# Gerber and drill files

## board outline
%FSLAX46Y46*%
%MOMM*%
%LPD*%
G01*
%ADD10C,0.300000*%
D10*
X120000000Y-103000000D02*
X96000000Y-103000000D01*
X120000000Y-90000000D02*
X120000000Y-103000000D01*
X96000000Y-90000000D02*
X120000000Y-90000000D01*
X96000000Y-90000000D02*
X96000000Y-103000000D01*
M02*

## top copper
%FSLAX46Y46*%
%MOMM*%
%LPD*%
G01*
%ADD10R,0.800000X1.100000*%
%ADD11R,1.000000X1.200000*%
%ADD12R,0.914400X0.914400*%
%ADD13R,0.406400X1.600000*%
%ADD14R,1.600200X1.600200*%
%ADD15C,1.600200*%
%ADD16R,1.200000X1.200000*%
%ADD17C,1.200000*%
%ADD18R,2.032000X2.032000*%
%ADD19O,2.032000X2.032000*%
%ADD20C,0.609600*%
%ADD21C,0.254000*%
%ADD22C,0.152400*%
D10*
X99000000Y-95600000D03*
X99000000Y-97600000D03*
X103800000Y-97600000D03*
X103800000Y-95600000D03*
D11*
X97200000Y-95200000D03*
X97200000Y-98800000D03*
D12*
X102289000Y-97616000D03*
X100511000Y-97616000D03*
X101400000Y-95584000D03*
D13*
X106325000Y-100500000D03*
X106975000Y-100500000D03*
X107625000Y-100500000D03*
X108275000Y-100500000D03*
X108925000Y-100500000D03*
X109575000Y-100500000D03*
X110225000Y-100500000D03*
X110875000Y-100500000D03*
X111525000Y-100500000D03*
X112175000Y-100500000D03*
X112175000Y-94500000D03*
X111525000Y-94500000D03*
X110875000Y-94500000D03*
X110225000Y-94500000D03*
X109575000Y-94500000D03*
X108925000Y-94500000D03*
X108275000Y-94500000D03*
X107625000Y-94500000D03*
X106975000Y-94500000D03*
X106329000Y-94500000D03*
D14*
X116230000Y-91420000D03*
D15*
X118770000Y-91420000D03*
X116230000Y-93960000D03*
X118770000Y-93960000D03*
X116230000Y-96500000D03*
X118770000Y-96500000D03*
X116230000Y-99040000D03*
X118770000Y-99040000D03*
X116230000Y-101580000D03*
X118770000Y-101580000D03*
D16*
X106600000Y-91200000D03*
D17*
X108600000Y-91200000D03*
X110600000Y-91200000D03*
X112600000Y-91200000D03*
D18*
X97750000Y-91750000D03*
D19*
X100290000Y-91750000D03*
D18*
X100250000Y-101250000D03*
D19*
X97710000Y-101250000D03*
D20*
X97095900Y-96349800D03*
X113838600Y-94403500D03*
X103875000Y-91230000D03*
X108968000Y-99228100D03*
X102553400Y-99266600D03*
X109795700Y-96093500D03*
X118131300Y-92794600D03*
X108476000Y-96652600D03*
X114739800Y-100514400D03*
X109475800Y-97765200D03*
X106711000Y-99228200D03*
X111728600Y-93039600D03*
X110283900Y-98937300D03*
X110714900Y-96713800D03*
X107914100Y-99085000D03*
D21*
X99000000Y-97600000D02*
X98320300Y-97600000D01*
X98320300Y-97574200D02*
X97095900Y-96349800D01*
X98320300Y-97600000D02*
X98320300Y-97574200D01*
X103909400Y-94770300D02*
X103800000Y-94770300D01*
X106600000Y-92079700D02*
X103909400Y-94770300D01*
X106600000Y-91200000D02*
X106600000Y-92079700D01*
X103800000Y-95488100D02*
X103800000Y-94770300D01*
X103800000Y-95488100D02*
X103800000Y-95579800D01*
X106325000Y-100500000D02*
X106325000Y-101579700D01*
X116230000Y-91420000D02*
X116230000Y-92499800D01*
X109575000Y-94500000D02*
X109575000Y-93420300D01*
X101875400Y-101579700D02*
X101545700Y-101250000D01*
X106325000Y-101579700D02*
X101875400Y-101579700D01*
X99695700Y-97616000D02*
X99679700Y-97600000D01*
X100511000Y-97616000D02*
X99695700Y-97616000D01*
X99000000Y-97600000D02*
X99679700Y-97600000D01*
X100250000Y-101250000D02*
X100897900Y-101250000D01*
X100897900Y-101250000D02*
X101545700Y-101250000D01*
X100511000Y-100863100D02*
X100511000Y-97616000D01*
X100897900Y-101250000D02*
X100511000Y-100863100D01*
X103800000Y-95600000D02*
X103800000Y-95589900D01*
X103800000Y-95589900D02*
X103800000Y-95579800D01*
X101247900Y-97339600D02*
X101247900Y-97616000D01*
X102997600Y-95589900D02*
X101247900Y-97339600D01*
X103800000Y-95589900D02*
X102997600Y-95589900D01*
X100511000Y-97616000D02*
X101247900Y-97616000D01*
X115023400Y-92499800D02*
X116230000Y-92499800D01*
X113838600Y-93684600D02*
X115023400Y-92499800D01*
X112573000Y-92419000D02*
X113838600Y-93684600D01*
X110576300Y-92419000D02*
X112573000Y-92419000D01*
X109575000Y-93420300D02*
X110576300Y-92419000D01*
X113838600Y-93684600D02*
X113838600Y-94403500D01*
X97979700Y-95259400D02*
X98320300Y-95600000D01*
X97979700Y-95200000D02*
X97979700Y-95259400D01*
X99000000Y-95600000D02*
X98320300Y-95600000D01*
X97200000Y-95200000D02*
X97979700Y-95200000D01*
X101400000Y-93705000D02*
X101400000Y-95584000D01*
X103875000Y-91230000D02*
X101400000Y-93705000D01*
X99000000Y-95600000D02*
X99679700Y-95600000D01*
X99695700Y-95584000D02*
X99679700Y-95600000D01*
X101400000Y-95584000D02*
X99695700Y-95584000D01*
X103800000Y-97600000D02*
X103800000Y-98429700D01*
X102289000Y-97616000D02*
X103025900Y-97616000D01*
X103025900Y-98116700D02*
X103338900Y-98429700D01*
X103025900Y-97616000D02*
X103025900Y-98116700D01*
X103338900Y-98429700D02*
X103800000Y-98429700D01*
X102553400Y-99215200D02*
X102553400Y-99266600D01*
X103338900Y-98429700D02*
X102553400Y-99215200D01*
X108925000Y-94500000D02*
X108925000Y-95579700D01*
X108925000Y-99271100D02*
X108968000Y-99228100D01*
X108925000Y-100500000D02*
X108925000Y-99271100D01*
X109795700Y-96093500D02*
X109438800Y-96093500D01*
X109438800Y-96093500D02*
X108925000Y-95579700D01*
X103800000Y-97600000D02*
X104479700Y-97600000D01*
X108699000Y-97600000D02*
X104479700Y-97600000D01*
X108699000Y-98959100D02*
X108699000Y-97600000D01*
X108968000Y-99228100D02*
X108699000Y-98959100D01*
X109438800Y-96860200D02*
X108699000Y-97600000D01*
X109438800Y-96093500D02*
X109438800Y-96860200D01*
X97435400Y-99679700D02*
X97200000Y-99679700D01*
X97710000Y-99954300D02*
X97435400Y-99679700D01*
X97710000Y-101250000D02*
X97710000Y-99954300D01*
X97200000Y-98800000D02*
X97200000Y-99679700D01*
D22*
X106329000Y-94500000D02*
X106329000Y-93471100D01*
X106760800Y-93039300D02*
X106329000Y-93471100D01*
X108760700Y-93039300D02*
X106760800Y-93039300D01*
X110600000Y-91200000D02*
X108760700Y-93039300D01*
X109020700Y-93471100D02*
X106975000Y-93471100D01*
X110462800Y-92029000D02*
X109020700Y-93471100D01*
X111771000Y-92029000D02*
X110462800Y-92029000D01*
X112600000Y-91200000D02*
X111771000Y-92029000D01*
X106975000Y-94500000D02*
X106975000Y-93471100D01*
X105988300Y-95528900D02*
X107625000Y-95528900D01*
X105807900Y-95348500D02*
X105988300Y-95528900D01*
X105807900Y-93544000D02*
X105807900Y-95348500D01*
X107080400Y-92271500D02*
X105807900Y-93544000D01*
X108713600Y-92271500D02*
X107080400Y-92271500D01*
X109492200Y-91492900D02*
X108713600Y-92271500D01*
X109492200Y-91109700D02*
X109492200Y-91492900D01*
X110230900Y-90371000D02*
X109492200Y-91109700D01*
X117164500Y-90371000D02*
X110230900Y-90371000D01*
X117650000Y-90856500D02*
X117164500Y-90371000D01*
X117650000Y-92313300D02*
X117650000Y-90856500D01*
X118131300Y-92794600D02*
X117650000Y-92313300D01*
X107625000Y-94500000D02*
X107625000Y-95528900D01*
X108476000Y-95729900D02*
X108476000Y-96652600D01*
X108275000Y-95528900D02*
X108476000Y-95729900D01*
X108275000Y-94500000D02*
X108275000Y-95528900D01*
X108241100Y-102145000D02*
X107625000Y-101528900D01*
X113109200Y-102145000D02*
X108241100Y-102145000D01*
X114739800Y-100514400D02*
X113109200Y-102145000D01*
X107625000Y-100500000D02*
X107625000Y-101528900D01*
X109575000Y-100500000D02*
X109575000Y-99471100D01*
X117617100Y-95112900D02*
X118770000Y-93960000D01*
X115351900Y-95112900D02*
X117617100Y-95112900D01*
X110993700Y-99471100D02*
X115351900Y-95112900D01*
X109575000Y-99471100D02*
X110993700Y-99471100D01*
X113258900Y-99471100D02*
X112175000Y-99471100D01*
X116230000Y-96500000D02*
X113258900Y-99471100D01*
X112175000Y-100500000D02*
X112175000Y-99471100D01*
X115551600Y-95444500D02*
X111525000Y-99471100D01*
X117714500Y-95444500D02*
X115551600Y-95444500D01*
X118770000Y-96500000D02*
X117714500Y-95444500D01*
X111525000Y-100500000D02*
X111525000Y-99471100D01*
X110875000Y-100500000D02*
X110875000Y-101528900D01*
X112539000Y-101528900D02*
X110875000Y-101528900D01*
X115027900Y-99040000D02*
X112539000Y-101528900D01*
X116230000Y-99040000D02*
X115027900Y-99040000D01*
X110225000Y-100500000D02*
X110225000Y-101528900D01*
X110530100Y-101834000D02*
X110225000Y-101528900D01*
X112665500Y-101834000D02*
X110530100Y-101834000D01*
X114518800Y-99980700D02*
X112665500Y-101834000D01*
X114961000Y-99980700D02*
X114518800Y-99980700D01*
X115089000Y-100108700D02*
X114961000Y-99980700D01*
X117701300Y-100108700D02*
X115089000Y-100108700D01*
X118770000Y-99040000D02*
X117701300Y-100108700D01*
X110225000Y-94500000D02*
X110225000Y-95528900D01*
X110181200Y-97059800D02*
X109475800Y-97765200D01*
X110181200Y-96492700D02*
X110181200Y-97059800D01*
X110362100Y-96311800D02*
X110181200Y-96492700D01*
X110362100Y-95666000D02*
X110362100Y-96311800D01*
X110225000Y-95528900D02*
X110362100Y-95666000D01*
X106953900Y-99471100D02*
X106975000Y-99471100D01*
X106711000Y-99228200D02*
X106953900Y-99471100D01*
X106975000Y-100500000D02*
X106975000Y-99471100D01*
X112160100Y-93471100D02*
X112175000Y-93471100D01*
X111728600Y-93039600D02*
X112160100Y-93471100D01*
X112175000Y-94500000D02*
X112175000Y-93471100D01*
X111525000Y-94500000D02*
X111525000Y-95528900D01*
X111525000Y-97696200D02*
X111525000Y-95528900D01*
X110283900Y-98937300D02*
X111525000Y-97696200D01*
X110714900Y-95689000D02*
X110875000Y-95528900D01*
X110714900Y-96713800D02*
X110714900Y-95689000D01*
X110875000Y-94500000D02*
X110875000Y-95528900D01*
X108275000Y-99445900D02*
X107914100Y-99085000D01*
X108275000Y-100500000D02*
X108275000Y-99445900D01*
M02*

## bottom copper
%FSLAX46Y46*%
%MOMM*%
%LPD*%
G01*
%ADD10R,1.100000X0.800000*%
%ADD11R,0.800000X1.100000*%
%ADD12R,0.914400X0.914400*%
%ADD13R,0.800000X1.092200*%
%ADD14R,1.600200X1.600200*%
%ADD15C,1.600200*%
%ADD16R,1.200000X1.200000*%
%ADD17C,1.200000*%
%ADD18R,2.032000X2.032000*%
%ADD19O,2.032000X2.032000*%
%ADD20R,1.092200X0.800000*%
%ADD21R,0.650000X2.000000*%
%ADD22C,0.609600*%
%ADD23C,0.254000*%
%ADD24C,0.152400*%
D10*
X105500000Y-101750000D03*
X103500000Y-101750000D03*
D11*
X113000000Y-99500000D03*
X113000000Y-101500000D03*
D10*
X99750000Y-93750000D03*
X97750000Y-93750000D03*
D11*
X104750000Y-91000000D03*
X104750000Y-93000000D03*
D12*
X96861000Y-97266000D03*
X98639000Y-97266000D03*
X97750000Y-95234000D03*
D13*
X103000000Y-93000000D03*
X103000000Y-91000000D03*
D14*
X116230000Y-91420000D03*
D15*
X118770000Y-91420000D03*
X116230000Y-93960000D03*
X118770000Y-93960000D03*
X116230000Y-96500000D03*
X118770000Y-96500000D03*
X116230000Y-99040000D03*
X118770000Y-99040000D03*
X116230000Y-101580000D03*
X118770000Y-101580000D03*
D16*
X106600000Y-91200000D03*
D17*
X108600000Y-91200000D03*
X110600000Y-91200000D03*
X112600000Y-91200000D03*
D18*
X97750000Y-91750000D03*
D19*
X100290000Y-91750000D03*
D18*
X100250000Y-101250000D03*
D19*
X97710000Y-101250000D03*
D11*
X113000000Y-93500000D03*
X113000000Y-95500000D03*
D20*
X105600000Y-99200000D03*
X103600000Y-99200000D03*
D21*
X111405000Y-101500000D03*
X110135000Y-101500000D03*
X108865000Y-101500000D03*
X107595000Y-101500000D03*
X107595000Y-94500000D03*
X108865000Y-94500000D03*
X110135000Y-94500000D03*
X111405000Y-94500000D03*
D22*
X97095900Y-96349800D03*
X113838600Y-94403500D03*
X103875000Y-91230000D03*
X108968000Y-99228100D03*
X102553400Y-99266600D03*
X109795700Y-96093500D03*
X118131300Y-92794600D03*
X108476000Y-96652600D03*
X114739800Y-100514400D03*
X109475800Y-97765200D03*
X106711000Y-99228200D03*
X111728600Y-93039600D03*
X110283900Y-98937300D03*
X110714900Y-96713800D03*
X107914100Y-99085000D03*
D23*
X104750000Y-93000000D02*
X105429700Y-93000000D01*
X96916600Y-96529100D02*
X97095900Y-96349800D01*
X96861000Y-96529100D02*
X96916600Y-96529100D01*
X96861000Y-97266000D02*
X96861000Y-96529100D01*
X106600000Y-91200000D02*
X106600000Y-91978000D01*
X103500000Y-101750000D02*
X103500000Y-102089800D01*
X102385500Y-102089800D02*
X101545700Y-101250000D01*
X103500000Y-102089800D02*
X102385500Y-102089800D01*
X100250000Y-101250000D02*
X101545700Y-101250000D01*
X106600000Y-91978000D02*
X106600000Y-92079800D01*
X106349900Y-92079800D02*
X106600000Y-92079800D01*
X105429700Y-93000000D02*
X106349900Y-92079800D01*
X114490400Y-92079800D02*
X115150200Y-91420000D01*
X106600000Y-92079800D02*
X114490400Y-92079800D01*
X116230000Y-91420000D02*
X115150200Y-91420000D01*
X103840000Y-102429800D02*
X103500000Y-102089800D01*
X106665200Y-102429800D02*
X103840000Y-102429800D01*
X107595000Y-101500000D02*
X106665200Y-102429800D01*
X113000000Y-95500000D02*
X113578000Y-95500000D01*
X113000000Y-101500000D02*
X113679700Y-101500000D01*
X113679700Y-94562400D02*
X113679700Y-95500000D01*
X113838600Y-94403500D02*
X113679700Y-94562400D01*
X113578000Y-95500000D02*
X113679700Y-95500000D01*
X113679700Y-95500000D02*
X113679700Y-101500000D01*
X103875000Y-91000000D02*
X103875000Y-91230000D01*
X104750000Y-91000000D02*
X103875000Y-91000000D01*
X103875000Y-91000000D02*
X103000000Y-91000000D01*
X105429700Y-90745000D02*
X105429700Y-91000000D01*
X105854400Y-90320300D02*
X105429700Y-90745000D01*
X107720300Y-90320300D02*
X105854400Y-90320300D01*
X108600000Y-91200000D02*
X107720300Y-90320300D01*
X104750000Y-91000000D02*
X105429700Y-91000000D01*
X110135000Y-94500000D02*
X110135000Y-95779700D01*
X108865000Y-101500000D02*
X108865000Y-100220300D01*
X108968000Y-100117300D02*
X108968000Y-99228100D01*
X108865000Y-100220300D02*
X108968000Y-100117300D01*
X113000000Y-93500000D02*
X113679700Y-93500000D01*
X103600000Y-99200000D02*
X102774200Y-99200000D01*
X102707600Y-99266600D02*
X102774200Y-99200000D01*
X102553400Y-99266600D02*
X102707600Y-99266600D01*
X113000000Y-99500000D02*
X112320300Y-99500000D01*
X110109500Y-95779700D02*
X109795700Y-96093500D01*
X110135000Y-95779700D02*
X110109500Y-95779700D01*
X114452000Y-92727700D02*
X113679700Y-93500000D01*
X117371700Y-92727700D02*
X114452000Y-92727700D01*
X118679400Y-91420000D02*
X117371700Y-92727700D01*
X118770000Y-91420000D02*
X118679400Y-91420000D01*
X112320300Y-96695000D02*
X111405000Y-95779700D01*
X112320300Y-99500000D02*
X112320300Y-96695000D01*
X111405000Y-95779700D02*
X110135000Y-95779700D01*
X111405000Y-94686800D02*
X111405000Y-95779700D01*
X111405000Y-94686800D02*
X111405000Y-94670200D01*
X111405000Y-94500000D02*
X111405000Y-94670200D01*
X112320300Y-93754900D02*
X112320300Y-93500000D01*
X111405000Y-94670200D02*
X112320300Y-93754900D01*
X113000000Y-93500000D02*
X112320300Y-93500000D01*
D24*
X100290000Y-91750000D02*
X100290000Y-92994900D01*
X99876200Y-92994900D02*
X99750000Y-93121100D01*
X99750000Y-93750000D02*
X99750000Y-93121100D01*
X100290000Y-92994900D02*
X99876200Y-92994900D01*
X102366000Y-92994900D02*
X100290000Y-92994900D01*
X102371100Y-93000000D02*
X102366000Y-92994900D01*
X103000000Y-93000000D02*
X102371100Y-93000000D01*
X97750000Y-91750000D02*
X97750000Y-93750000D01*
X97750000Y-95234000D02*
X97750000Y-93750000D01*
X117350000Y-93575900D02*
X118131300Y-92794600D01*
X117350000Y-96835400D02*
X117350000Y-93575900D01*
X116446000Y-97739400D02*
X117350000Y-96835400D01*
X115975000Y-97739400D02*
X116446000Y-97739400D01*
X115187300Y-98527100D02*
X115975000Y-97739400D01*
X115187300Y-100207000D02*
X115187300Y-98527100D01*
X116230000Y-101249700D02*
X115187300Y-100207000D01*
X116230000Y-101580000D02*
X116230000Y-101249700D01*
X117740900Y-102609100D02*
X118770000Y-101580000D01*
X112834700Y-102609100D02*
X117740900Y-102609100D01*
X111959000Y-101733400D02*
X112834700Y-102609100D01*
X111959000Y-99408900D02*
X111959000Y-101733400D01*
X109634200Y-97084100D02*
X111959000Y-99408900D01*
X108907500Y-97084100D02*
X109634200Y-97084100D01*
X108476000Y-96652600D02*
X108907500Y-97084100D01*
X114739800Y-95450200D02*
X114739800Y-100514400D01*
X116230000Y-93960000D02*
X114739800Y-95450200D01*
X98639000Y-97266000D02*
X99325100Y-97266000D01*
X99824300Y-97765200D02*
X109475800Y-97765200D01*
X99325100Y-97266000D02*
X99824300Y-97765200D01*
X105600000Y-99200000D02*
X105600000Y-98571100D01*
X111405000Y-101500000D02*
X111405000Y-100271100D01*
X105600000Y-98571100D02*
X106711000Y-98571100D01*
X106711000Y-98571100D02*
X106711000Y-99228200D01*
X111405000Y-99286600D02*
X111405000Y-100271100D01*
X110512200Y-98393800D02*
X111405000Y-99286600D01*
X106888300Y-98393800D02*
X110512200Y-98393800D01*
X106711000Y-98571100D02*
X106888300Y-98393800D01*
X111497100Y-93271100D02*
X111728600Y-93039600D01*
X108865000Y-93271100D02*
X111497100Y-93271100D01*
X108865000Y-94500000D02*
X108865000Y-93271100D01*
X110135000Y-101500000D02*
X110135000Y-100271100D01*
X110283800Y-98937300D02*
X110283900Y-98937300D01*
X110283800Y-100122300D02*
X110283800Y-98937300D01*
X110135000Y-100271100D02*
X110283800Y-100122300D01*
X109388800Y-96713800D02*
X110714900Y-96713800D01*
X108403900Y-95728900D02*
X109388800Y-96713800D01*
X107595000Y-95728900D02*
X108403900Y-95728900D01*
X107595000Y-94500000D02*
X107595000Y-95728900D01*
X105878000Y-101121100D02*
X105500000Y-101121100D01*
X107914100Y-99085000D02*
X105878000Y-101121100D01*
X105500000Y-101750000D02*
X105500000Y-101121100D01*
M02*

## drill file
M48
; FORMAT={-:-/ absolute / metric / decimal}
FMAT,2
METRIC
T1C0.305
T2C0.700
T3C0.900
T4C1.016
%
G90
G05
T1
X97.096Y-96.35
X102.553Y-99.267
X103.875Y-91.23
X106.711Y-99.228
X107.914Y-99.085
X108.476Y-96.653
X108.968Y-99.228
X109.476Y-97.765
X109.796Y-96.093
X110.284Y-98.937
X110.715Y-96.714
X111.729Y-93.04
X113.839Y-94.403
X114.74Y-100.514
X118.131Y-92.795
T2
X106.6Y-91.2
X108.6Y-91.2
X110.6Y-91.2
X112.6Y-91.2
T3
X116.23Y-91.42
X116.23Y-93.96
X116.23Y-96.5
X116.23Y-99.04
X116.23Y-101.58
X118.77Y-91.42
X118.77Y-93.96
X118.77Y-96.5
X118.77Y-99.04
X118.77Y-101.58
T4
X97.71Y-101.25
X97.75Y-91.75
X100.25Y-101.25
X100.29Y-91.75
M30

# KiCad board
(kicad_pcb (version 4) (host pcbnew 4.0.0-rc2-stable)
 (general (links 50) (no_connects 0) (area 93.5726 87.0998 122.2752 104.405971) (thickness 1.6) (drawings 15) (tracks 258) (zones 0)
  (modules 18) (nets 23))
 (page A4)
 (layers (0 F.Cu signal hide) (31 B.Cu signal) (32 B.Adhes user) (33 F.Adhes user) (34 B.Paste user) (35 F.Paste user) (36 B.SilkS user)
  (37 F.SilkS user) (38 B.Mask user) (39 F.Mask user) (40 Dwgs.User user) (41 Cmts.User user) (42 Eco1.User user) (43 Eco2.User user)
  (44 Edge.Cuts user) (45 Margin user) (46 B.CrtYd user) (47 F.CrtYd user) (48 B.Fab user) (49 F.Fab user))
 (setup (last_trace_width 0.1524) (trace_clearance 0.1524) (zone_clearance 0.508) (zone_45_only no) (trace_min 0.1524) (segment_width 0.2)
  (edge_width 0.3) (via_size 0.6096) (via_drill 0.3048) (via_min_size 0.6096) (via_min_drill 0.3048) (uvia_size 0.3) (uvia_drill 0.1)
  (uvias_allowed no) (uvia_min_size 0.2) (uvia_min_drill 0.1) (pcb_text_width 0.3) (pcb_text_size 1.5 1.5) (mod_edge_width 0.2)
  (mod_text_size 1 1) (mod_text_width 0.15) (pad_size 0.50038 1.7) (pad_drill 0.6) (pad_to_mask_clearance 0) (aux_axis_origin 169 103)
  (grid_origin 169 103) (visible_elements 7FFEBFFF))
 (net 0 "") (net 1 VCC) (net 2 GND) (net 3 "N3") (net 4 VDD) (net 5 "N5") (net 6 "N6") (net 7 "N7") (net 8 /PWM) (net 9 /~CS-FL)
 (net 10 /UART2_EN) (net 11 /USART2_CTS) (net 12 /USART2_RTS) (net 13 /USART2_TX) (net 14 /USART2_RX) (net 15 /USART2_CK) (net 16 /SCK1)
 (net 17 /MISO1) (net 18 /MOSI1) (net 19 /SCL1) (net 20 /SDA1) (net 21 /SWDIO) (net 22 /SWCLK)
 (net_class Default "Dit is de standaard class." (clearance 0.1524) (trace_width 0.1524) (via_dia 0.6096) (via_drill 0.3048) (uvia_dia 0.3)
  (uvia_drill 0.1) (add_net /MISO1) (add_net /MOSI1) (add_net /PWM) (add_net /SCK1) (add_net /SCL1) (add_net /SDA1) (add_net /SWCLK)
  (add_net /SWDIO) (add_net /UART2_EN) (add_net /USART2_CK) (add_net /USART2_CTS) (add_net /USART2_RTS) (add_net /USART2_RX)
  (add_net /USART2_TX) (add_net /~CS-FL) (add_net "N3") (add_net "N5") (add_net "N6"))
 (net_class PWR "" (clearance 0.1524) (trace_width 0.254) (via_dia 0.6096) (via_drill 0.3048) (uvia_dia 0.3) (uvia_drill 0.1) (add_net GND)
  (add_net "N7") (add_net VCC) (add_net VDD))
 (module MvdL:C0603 (layer F.Cu) (at 99 96.6 270)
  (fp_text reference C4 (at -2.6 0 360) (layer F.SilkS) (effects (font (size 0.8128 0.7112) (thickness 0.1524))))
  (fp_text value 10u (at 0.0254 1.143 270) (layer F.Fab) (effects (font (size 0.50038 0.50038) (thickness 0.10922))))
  (pad 1 smd rect (at -1 0 270) (size 1.1 0.8) (layers F.Cu F.Paste F.Mask) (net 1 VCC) (clearance 0.1524))
  (pad 2 smd rect (at 1 0 270) (size 1.1 0.8) (layers F.Cu F.Paste F.Mask) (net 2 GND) (clearance 0.1524)))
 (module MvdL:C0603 (layer B.Cu) (at 104.5 101.75 180)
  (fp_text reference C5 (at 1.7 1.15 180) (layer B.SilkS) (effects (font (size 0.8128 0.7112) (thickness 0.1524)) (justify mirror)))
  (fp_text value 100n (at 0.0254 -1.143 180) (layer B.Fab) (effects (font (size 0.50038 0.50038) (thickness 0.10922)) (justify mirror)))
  (pad 1 smd rect (at -1 0 180) (size 1.1 0.8) (layers B.Cu B.Paste B.Mask) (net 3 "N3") (clearance 0.1524))
  (pad 2 smd rect (at 1 0 180) (size 1.1 0.8) (layers B.Cu B.Paste B.Mask) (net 2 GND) (clearance 0.1524)))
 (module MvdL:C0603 (layer F.Cu) (at 103.8 96.6 90)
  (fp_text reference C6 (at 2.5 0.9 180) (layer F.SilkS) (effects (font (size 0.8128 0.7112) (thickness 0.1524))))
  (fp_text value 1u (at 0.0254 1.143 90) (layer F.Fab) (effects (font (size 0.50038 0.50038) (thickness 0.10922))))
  (pad 1 smd rect (at -1 0 90) (size 1.1 0.8) (layers F.Cu F.Paste F.Mask) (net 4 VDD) (clearance 0.1524))
  (pad 2 smd rect (at 1 0 90) (size 1.1 0.8) (layers F.Cu F.Paste F.Mask) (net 2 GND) (clearance 0.1524)))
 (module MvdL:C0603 (layer B.Cu) (at 113 100.5 270)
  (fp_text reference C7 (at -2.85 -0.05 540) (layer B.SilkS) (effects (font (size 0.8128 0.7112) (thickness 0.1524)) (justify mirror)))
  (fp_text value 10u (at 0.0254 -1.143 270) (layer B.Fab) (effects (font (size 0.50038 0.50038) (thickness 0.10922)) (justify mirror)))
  (pad 1 smd rect (at -1 0 270) (size 1.1 0.8) (layers B.Cu B.Paste B.Mask) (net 4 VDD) (clearance 0.1524))
  (pad 2 smd rect (at 1 0 270) (size 1.1 0.8) (layers B.Cu B.Paste B.Mask) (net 2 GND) (clearance 0.1524)))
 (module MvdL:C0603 (layer B.Cu) (at 98.75 93.75 180)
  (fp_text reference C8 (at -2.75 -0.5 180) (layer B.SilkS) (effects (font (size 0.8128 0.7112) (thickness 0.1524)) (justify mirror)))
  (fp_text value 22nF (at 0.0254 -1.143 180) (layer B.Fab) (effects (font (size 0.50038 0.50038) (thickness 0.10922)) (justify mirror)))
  (pad 1 smd rect (at -1 0 180) (size 1.1 0.8) (layers B.Cu B.Paste B.Mask) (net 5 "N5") (clearance 0.1524))
  (pad 2 smd rect (at 1 0 180) (size 1.1 0.8) (layers B.Cu B.Paste B.Mask) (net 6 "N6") (clearance 0.1524)))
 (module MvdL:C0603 (layer B.Cu) (at 104.75 92 270)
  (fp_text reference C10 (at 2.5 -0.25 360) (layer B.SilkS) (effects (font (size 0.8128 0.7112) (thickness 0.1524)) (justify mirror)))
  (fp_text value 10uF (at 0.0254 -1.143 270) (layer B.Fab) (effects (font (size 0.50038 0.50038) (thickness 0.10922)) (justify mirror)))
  (pad 1 smd rect (at -1 0 270) (size 1.1 0.8) (layers B.Cu B.Paste B.Mask) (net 1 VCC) (clearance 0.1524))
  (pad 2 smd rect (at 1 0 270) (size 1.1 0.8) (layers B.Cu B.Paste B.Mask) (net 2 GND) (clearance 0.1524)))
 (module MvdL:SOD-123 (layer F.Cu) (at 97.2 97 270)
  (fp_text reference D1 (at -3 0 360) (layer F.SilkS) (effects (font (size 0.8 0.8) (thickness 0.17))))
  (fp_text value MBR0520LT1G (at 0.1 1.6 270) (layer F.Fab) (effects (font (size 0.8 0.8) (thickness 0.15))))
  (pad C smd rect (at -1.8 0 270) (size 1.2 1) (layers F.Cu F.Paste F.Mask) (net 1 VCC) (clearance 0.1524))
  (pad A smd rect (at 1.8 0 270) (size 1.2 1) (layers F.Cu F.Paste F.Mask) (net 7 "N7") (clearance 0.1524)))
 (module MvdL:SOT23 (layer B.Cu) (at 97.75 96.25)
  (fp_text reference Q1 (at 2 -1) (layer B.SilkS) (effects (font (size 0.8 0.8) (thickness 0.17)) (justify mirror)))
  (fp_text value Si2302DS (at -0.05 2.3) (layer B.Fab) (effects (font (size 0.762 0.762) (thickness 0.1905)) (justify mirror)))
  (pad 2 smd rect (at -0.889 1.016) (size 0.9144 0.9144) (layers B.Cu B.Paste B.Mask) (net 2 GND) (die_length -2147.483648)
   (clearance 0.1524))
  (pad 1 smd rect (at 0.889 1.016) (size 0.9144 0.9144) (layers B.Cu B.Paste B.Mask) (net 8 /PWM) (clearance 0.1524))
  (pad 3 smd rect (at 0 -1.016) (size 0.9144 0.9144) (layers B.Cu B.Paste B.Mask) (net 6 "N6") (clearance 0.1524)))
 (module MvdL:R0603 (layer B.Cu) (at 103 92 90)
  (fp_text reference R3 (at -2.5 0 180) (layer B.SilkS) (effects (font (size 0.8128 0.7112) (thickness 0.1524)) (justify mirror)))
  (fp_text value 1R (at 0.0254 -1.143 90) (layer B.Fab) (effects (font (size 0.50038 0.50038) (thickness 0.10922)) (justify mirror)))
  (pad 1 smd rect (at -1 0 90) (size 1.0922 0.8) (layers B.Cu B.Paste B.Mask) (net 5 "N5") (clearance 0.1524))
  (pad 2 smd rect (at 1 0 90) (size 1.0922 0.8) (layers B.Cu B.Paste B.Mask) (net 1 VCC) (clearance 0.1524)))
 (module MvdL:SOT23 (layer F.Cu) (at 101.4 96.6 180)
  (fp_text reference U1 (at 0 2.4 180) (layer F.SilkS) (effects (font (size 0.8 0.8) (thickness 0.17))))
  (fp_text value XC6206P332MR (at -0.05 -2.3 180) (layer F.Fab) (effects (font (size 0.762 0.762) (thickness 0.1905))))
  (pad 2 smd rect (at -0.889 -1.016 180) (size 0.9144 0.9144) (layers F.Cu F.Paste F.Mask) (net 4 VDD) (die_length -2147.483648)
   (clearance 0.1524))
  (pad 1 smd rect (at 0.889 -1.016 180) (size 0.9144 0.9144) (layers F.Cu F.Paste F.Mask) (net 2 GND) (clearance 0.1524))
  (pad 3 smd rect (at 0 1.016 180) (size 0.9144 0.9144) (layers F.Cu F.Paste F.Mask) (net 1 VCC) (clearance 0.1524)))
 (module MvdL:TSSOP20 (layer F.Cu) (at 109.25 97.5)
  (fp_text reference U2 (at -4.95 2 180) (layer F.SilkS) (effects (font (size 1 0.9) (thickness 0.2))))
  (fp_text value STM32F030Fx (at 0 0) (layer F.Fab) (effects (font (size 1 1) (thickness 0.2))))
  (pad 1 smd rect (at -2.925 3) (size 0.4064 1.6) (layers F.Cu F.Paste F.Mask) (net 2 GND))
  (pad 2 smd rect (at -2.275 3) (size 0.4064 1.6) (layers F.Cu F.Paste F.Mask) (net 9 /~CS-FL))
  (pad 3 smd rect (at -1.625 3) (size 0.4064 1.6) (layers F.Cu F.Paste F.Mask) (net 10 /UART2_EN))
  (pad 4 smd rect (at -0.975 3) (size 0.4064 1.6) (layers F.Cu F.Paste F.Mask) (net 3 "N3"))
  (pad 5 smd rect (at -0.325 3) (size 0.4064 1.6) (layers F.Cu F.Paste F.Mask) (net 4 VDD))
  (pad 6 smd rect (at 0.325 3) (size 0.4064 1.6) (layers F.Cu F.Paste F.Mask) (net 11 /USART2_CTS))
  (pad 7 smd rect (at 0.975 3) (size 0.4064 1.6) (layers F.Cu F.Paste F.Mask) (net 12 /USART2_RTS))
  (pad 8 smd rect (at 1.625 3) (size 0.4064 1.6) (layers F.Cu F.Paste F.Mask) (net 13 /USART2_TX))
  (pad 9 smd rect (at 2.275 3) (size 0.4064 1.6) (layers F.Cu F.Paste F.Mask) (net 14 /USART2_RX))
  (pad 10 smd rect (at 2.925 3) (size 0.4064 1.6) (layers F.Cu F.Paste F.Mask) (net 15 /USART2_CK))
  (pad 11 smd rect (at 2.925 -3) (size 0.4064 1.6) (layers F.Cu F.Paste F.Mask) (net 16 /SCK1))
  (pad 12 smd rect (at 2.275 -3) (size 0.4064 1.6) (layers F.Cu F.Paste F.Mask) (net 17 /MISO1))
  (pad 13 smd rect (at 1.625 -3) (size 0.4064 1.6) (layers F.Cu F.Paste F.Mask) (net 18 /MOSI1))
  (pad 14 smd rect (at 0.975 -3) (size 0.4064 1.6) (layers F.Cu F.Paste F.Mask) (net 8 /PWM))
  (pad 15 smd rect (at 0.325 -3) (size 0.4064 1.6) (layers F.Cu F.Paste F.Mask) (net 2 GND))
  (pad 16 smd rect (at -0.325 -3) (size 0.4064 1.6) (layers F.Cu F.Paste F.Mask) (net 4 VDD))
  (pad 17 smd rect (at -0.975 -3) (size 0.4064 1.6) (layers F.Cu F.Paste F.Mask) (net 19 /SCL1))
  (pad 18 smd rect (at -1.625 -3) (size 0.4064 1.6) (layers F.Cu F.Paste F.Mask) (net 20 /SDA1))
  (pad 19 smd rect (at -2.275 -3) (size 0.4064 1.6) (layers F.Cu F.Paste F.Mask) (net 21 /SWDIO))
  (pad 20 smd rect (at -2.921 -3) (size 0.4064 1.6) (layers F.Cu F.Paste F.Mask) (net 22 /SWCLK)))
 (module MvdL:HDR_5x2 (layer F.Cu) (at 117.5 96.5 270)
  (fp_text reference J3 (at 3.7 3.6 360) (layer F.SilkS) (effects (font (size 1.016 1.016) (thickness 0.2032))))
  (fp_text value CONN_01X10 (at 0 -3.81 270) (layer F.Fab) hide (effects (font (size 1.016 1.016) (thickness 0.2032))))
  (pad 1 thru_hole rect (at -5.08 1.27 270) (size 1.6002 1.6002) (drill 0.9) (layers *.Cu *.Mask F.SilkS) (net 2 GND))
  (pad 2 thru_hole circle (at -5.08 -1.27 270) (size 1.6002 1.6002) (drill 0.9) (layers *.Cu *.Mask F.SilkS) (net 4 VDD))
  (pad 3 thru_hole circle (at -2.54 1.27 270) (size 1.6002 1.6002) (drill 0.9) (layers *.Cu *.Mask F.SilkS) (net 10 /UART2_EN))
  (pad 4 thru_hole circle (at -2.54 -1.27 270) (size 1.6002 1.6002) (drill 0.9) (layers *.Cu *.Mask F.SilkS) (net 11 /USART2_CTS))
  (pad 5 thru_hole circle (at 0 1.27 270) (size 1.6002 1.6002) (drill 0.9) (layers *.Cu *.Mask F.SilkS) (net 15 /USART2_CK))
  (pad 6 thru_hole circle (at 0 -1.27 270) (size 1.6002 1.6002) (drill 0.9) (layers *.Cu *.Mask F.SilkS) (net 14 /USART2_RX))
  (pad 7 thru_hole circle (at 2.54 1.27 270) (size 1.6002 1.6002) (drill 0.9) (layers *.Cu *.Mask F.SilkS) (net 13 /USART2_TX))
  (pad 8 thru_hole circle (at 2.54 -1.27 270) (size 1.6002 1.6002) (drill 0.9) (layers *.Cu *.Mask F.SilkS) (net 12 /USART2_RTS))
  (pad 9 thru_hole circle (at 5.08 1.27 270) (size 1.6002 1.6002) (drill 0.9) (layers *.Cu *.Mask F.SilkS) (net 20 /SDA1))
  (pad 10 thru_hole circle (at 5.08 -1.27 270) (size 1.6002 1.6002) (drill 0.9) (layers *.Cu *.Mask F.SilkS) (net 19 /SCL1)))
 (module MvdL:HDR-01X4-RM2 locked (layer F.Cu) (at 106.6 91.2)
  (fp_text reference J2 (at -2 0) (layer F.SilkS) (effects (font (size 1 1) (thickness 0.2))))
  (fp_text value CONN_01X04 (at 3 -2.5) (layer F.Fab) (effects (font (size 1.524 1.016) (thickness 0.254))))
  (pad 1 thru_hole rect (at 0 0) (size 1.2 1.2) (drill 0.7) (layers *.Cu *.Mask F.SilkS) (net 2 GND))
  (pad 2 thru_hole circle (at 2 0) (size 1.2 1.2) (drill 0.7) (layers *.Cu *.Mask F.SilkS) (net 1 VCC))
  (pad 3 thru_hole circle (at 4 0) (size 1.2 1.2) (drill 0.7) (layers *.Cu *.Mask F.SilkS) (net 22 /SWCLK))
  (pad 4 thru_hole circle (at 6 0) (size 1.2 1.2) (drill 0.7) (layers *.Cu *.Mask F.SilkS) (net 21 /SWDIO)))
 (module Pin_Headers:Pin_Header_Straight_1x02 (layer F.Cu) (at 97.75 91.75 90)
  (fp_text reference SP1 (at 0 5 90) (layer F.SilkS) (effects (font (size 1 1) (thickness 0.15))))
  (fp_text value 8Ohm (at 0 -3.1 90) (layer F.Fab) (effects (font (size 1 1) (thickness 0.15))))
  (pad 1 thru_hole rect (at 0 0 90) (size 2.032 2.032) (drill 1.016) (layers *.Cu *.Mask F.SilkS) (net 6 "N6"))
  (pad 2 thru_hole oval (at 0 2.54 90) (size 2.032 2.032) (drill 1.016) (layers *.Cu *.Mask F.SilkS) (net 5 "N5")))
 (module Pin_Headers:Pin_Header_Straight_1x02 (layer F.Cu) (at 100.25 101.25 270)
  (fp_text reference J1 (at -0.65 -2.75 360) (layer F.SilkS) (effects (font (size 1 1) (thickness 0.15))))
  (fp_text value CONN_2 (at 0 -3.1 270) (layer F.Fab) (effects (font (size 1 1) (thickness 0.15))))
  (pad 1 thru_hole rect (at 0 0 270) (size 2.032 2.032) (drill 1.016) (layers *.Cu *.Mask F.SilkS) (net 2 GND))
  (pad 2 thru_hole oval (at 0 2.54 270) (size 2.032 2.032) (drill 1.016) (layers *.Cu *.Mask F.SilkS) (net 7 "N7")))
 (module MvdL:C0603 (layer B.Cu) (at 113 94.5 270)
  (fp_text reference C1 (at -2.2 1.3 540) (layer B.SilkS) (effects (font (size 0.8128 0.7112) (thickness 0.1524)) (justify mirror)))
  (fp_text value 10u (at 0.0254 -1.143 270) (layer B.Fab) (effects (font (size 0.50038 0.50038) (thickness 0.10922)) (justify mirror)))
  (pad 1 smd rect (at -1 0 270) (size 1.1 0.8) (layers B.Cu B.Paste B.Mask) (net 4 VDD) (clearance 0.1524))
  (pad 2 smd rect (at 1 0 270) (size 1.1 0.8) (layers B.Cu B.Paste B.Mask) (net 2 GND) (clearance 0.1524)))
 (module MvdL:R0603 (layer B.Cu) (at 104.6 99.2 180)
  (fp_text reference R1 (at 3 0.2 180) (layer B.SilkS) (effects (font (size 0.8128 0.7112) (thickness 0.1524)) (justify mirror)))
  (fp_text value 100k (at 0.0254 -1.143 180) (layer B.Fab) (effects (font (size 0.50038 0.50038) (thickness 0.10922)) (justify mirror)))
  (pad 1 smd rect (at -1 0 180) (size 1.0922 0.8) (layers B.Cu B.Paste B.Mask) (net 9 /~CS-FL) (clearance 0.1524))
  (pad 2 smd rect (at 1 0 180) (size 1.0922 0.8) (layers B.Cu B.Paste B.Mask) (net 4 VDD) (clearance 0.1524)))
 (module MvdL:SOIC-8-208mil (layer B.Cu) (at 109.5 98 90)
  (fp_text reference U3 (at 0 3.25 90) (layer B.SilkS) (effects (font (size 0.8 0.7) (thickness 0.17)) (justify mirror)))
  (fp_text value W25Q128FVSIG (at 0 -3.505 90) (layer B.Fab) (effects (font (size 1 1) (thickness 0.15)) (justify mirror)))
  (pad 1 smd rect (at -3.5 1.905 90) (size 2 0.65) (layers B.Cu B.Paste B.Mask) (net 9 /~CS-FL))
  (pad 2 smd rect (at -3.5 0.635 90) (size 2 0.65) (layers B.Cu B.Paste B.Mask) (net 17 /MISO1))
  (pad 3 smd rect (at -3.5 -0.635 90) (size 2 0.65) (layers B.Cu B.Paste B.Mask) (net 4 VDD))
  (pad 4 smd rect (at -3.5 -1.905 90) (size 2 0.65) (layers B.Cu B.Paste B.Mask) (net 2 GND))
  (pad 5 smd rect (at 3.5 -1.905 90) (size 2 0.65) (layers B.Cu B.Paste B.Mask) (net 18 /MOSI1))
  (pad 6 smd rect (at 3.5 -0.635 90) (size 2 0.65) (layers B.Cu B.Paste B.Mask) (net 16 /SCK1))
  (pad 7 smd rect (at 3.5 0.635 90) (size 2 0.65) (layers B.Cu B.Paste B.Mask) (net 4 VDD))
  (pad 8 smd rect (at 3.5 1.905 90) (size 2 0.65) (layers B.Cu B.Paste B.Mask) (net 4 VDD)))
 (gr_line (start 120 103) (end 96 103) (angle 90) (layer Edge.Cuts) (width 0.3))
 (gr_line (start 120 90) (end 120 103) (angle 90) (layer Edge.Cuts) (width 0.3))
 (gr_line (start 96 90) (end 120 90) (angle 90) (layer Edge.Cuts) (width 0.3))
 (gr_line (start 96 90) (end 96 103) (angle 90) (layer Edge.Cuts) (width 0.3))
 (via (at 97.0959 96.3498) (size 0.6096) (layers F.Cu B.Cu) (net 2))
 (via (at 113.8386 94.4035) (size 0.6096) (layers F.Cu B.Cu) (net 2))
 (segment (start 104.75 93) (end 105.4297 93) (width 0.254) (layer B.Cu) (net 2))
 (segment (start 99 97.6) (end 98.3203 97.6) (width 0.254) (layer F.Cu) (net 2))
 (segment (start 96.9166 96.5291) (end 97.0959 96.3498) (width 0.254) (layer B.Cu) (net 2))
 (segment (start 96.861 96.5291) (end 96.9166 96.5291) (width 0.254) (layer B.Cu) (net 2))
 (segment (start 98.3203 97.5742) (end 97.0959 96.3498) (width 0.254) (layer F.Cu) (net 2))
 (segment (start 98.3203 97.6) (end 98.3203 97.5742) (width 0.254) (layer F.Cu) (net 2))
 (segment (start 96.861 97.266) (end 96.861 96.5291) (width 0.254) (layer B.Cu) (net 2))
 (segment (start 103.9094 94.7703) (end 103.8 94.7703) (width 0.254) (layer F.Cu) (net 2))
 (segment (start 106.6 92.0797) (end 103.9094 94.7703) (width 0.254) (layer F.Cu) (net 2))
 (segment (start 106.6 91.2) (end 106.6 92.0797) (width 0.254) (layer F.Cu) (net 2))
 (segment (start 103.8 95.4881) (end 103.8 94.7703) (width 0.254) (layer F.Cu) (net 2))
 (segment (start 103.8 95.4881) (end 103.8 95.5798) (width 0.254) (layer F.Cu) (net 2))
 (segment (start 106.325 100.5) (end 106.325 101.5797) (width 0.254) (layer F.Cu) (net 2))
 (segment (start 106.6 91.2) (end 106.6 91.978) (width 0.254) (layer B.Cu) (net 2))
 (segment (start 116.23 91.42) (end 116.23 92.4998) (width 0.254) (layer F.Cu) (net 2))
 (segment (start 103.5 101.75) (end 103.5 102.0898) (width 0.254) (layer B.Cu) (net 2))
 (segment (start 102.3855 102.0898) (end 101.5457 101.25) (width 0.254) (layer B.Cu) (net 2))
 (segment (start 103.5 102.0898) (end 102.3855 102.0898) (width 0.254) (layer B.Cu) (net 2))
 (segment (start 100.25 101.25) (end 101.5457 101.25) (width 0.254) (layer B.Cu) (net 2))
 (segment (start 109.575 94.5) (end 109.575 93.4203) (width 0.254) (layer F.Cu) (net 2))
 (segment (start 106.6 91.978) (end 106.6 92.0798) (width 0.254) (layer B.Cu) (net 2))
 (segment (start 106.3499 92.0798) (end 106.6 92.0798) (width 0.254) (layer B.Cu) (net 2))
 (segment (start 105.4297 93) (end 106.3499 92.0798) (width 0.254) (layer B.Cu) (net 2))
 (segment (start 114.4904 92.0798) (end 115.1502 91.42) (width 0.254) (layer B.Cu) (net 2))
 (segment (start 106.6 92.0798) (end 114.4904 92.0798) (width 0.254) (layer B.Cu) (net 2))
 (segment (start 116.23 91.42) (end 115.1502 91.42) (width 0.254) (layer B.Cu) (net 2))
 (segment (start 103.84 102.4298) (end 103.5 102.0898) (width 0.254) (layer B.Cu) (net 2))
 (segment (start 106.6652 102.4298) (end 103.84 102.4298) (width 0.254) (layer B.Cu) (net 2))
 (segment (start 107.595 101.5) (end 106.6652 102.4298) (width 0.254) (layer B.Cu) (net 2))
 (segment (start 113 95.5) (end 113.578 95.5) (width 0.254) (layer B.Cu) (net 2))
 (segment (start 113 101.5) (end 113.6797 101.5) (width 0.254) (layer B.Cu) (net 2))
 (segment (start 101.8754 101.5797) (end 101.5457 101.25) (width 0.254) (layer F.Cu) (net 2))
 (segment (start 106.325 101.5797) (end 101.8754 101.5797) (width 0.254) (layer F.Cu) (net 2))
 (segment (start 99.6957 97.616) (end 99.6797 97.6) (width 0.254) (layer F.Cu) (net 2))
 (segment (start 100.511 97.616) (end 99.6957 97.616) (width 0.254) (layer F.Cu) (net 2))
 (segment (start 99 97.6) (end 99.6797 97.6) (width 0.254) (layer F.Cu) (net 2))
 (segment (start 100.25 101.25) (end 100.8979 101.25) (width 0.254) (layer F.Cu) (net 2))
 (segment (start 100.8979 101.25) (end 101.5457 101.25) (width 0.254) (layer F.Cu) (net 2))
 (segment (start 100.511 100.8631) (end 100.511 97.616) (width 0.254) (layer F.Cu) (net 2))
 (segment (start 100.8979 101.25) (end 100.511 100.8631) (width 0.254) (layer F.Cu) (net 2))
 (segment (start 103.8 95.6) (end 103.8 95.5899) (width 0.254) (layer F.Cu) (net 2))
 (segment (start 103.8 95.5899) (end 103.8 95.5798) (width 0.254) (layer F.Cu) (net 2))
 (segment (start 101.2479 97.3396) (end 101.2479 97.616) (width 0.254) (layer F.Cu) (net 2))
 (segment (start 102.9976 95.5899) (end 101.2479 97.3396) (width 0.254) (layer F.Cu) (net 2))
 (segment (start 103.8 95.5899) (end 102.9976 95.5899) (width 0.254) (layer F.Cu) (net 2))
 (segment (start 100.511 97.616) (end 101.2479 97.616) (width 0.254) (layer F.Cu) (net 2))
 (segment (start 113.6797 94.5624) (end 113.6797 95.5) (width 0.254) (layer B.Cu) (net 2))
 (segment (start 113.8386 94.4035) (end 113.6797 94.5624) (width 0.254) (layer B.Cu) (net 2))
 (segment (start 113.578 95.5) (end 113.6797 95.5) (width 0.254) (layer B.Cu) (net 2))
 (segment (start 113.6797 95.5) (end 113.6797 101.5) (width 0.254) (layer B.Cu) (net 2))
 (segment (start 115.0234 92.4998) (end 116.23 92.4998) (width 0.254) (layer F.Cu) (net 2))
 (segment (start 113.8386 93.6846) (end 115.0234 92.4998) (width 0.254) (layer F.Cu) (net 2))
 (segment (start 112.573 92.419) (end 113.8386 93.6846) (width 0.254) (layer F.Cu) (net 2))
 (segment (start 110.5763 92.419) (end 112.573 92.419) (width 0.254) (layer F.Cu) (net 2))
 (segment (start 109.575 93.4203) (end 110.5763 92.419) (width 0.254) (layer F.Cu) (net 2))
 (segment (start 113.8386 93.6846) (end 113.8386 94.4035) (width 0.254) (layer F.Cu) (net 2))
 (via (at 103.875 91.23) (size 0.6096) (layers F.Cu B.Cu) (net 1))
 (segment (start 97.9797 95.2594) (end 98.3203 95.6) (width 0.254) (layer F.Cu) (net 1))
 (segment (start 97.9797 95.2) (end 97.9797 95.2594) (width 0.254) (layer F.Cu) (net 1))
 (segment (start 99 95.6) (end 98.3203 95.6) (width 0.254) (layer F.Cu) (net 1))
 (segment (start 97.2 95.2) (end 97.9797 95.2) (width 0.254) (layer F.Cu) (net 1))
 (segment (start 103.875 91) (end 103.875 91.23) (width 0.254) (layer B.Cu) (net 1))
 (segment (start 104.75 91) (end 103.875 91) (width 0.254) (layer B.Cu) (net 1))
 (segment (start 103.875 91) (end 103 91) (width 0.254) (layer B.Cu) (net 1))
 (segment (start 101.4 93.705) (end 101.4 95.584) (width 0.254) (layer F.Cu) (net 1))
 (segment (start 103.875 91.23) (end 101.4 93.705) (width 0.254) (layer F.Cu) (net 1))
 (segment (start 99 95.6) (end 99.6797 95.6) (width 0.254) (layer F.Cu) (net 1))
 (segment (start 99.6957 95.584) (end 99.6797 95.6) (width 0.254) (layer F.Cu) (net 1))
 (segment (start 101.4 95.584) (end 99.6957 95.584) (width 0.254) (layer F.Cu) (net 1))
 (segment (start 105.4297 90.745) (end 105.4297 91) (width 0.254) (layer B.Cu) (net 1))
 (segment (start 105.8544 90.3203) (end 105.4297 90.745) (width 0.254) (layer B.Cu) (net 1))
 (segment (start 107.7203 90.3203) (end 105.8544 90.3203) (width 0.254) (layer B.Cu) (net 1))
 (segment (start 108.6 91.2) (end 107.7203 90.3203) (width 0.254) (layer B.Cu) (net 1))
 (segment (start 104.75 91) (end 105.4297 91) (width 0.254) (layer B.Cu) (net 1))
 (via (at 108.968 99.2281) (size 0.6096) (layers F.Cu B.Cu) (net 4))
 (via (at 102.5534 99.2666) (size 0.6096) (layers F.Cu B.Cu) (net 4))
 (via (at 109.7957 96.0935) (size 0.6096) (layers F.Cu B.Cu) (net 4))
 (segment (start 110.135 94.5) (end 110.135 95.7797) (width 0.254) (layer B.Cu) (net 4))
 (segment (start 108.865 101.5) (end 108.865 100.2203) (width 0.254) (layer B.Cu) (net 4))
 (segment (start 108.968 100.1173) (end 108.968 99.2281) (width 0.254) (layer B.Cu) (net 4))
 (segment (start 108.865 100.2203) (end 108.968 100.1173) (width 0.254) (layer B.Cu) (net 4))
 (segment (start 113 93.5) (end 113.6797 93.5) (width 0.254) (layer B.Cu) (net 4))
 (segment (start 103.8 97.6) (end 103.8 98.4297) (width 0.254) (layer F.Cu) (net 4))
 (segment (start 102.289 97.616) (end 103.0259 97.616) (width 0.254) (layer F.Cu) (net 4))
 (segment (start 103.0259 98.1167) (end 103.3389 98.4297) (width 0.254) (layer F.Cu) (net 4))
 (segment (start 103.0259 97.616) (end 103.0259 98.1167) (width 0.254) (layer F.Cu) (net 4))
 (segment (start 103.3389 98.4297) (end 103.8 98.4297) (width 0.254) (layer F.Cu) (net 4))
 (segment (start 103.6 99.2) (end 102.7742 99.2) (width 0.254) (layer B.Cu) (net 4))
 (segment (start 102.7076 99.2666) (end 102.7742 99.2) (width 0.254) (layer B.Cu) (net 4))
 (segment (start 102.5534 99.2666) (end 102.7076 99.2666) (width 0.254) (layer B.Cu) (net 4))
 (segment (start 102.5534 99.2152) (end 102.5534 99.2666) (width 0.254) (layer F.Cu) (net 4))
 (segment (start 103.3389 98.4297) (end 102.5534 99.2152) (width 0.254) (layer F.Cu) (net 4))
 (segment (start 113 99.5) (end 112.3203 99.5) (width 0.254) (layer B.Cu) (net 4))
 (segment (start 110.1095 95.7797) (end 109.7957 96.0935) (width 0.254) (layer B.Cu) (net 4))
 (segment (start 110.135 95.7797) (end 110.1095 95.7797) (width 0.254) (layer B.Cu) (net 4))
 (segment (start 108.925 94.5) (end 108.925 95.5797) (width 0.254) (layer F.Cu) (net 4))
 (segment (start 108.925 99.2711) (end 108.968 99.2281) (width 0.254) (layer F.Cu) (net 4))
 (segment (start 108.925 100.5) (end 108.925 99.2711) (width 0.254) (layer F.Cu) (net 4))
 (segment (start 109.7957 96.0935) (end 109.4388 96.0935) (width 0.254) (layer F.Cu) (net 4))
 (segment (start 109.4388 96.0935) (end 108.925 95.5797) (width 0.254) (layer F.Cu) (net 4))
 (segment (start 103.8 97.6) (end 104.4797 97.6) (width 0.254) (layer F.Cu) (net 4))
 (segment (start 108.699 97.6) (end 104.4797 97.6) (width 0.254) (layer F.Cu) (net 4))
 (segment (start 108.699 98.9591) (end 108.699 97.6) (width 0.254) (layer F.Cu) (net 4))
 (segment (start 108.968 99.2281) (end 108.699 98.9591) (width 0.254) (layer F.Cu) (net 4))
 (segment (start 114.452 92.7277) (end 113.6797 93.5) (width 0.254) (layer B.Cu) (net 4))
 (segment (start 117.3717 92.7277) (end 114.452 92.7277) (width 0.254) (layer B.Cu) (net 4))
 (segment (start 118.6794 91.42) (end 117.3717 92.7277) (width 0.254) (layer B.Cu) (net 4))
 (segment (start 118.77 91.42) (end 118.6794 91.42) (width 0.254) (layer B.Cu) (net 4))
 (segment (start 109.4388 96.8602) (end 108.699 97.6) (width 0.254) (layer F.Cu) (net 4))
 (segment (start 109.4388 96.0935) (end 109.4388 96.8602) (width 0.254) (layer F.Cu) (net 4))
 (segment (start 112.3203 96.695) (end 111.405 95.7797) (width 0.254) (layer B.Cu) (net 4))
 (segment (start 112.3203 99.5) (end 112.3203 96.695) (width 0.254) (layer B.Cu) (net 4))
 (segment (start 111.405 95.7797) (end 110.135 95.7797) (width 0.254) (layer B.Cu) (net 4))
 (segment (start 111.405 94.6868) (end 111.405 95.7797) (width 0.254) (layer B.Cu) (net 4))
 (segment (start 111.405 94.6868) (end 111.405 94.6702) (width 0.254) (layer B.Cu) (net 4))
 (segment (start 111.405 94.5) (end 111.405 94.6702) (width 0.254) (layer B.Cu) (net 4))
 (segment (start 112.3203 93.7549) (end 112.3203 93.5) (width 0.254) (layer B.Cu) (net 4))
 (segment (start 111.405 94.6702) (end 112.3203 93.7549) (width 0.254) (layer B.Cu) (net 4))
 (segment (start 113 93.5) (end 112.3203 93.5) (width 0.254) (layer B.Cu) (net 4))
 (segment (start 100.29 91.75) (end 100.29 92.9949) (width 0.1524) (layer B.Cu) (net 5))
 (segment (start 99.8762 92.9949) (end 99.75 93.1211) (width 0.1524) (layer B.Cu) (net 5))
 (segment (start 99.75 93.75) (end 99.75 93.1211) (width 0.1524) (layer B.Cu) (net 5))
 (segment (start 100.29 92.9949) (end 99.8762 92.9949) (width 0.1524) (layer B.Cu) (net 5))
 (segment (start 102.366 92.9949) (end 100.29 92.9949) (width 0.1524) (layer B.Cu) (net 5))
 (segment (start 102.3711 93) (end 102.366 92.9949) (width 0.1524) (layer B.Cu) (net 5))
 (segment (start 103 93) (end 102.3711 93) (width 0.1524) (layer B.Cu) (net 5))
 (segment (start 97.75 91.75) (end 97.75 93.75) (width 0.1524) (layer B.Cu) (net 6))
 (segment (start 97.75 95.234) (end 97.75 93.75) (width 0.1524) (layer B.Cu) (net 6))
 (segment (start 97.4354 99.6797) (end 97.2 99.6797) (width 0.254) (layer F.Cu) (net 7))
 (segment (start 97.71 99.9543) (end 97.4354 99.6797) (width 0.254) (layer F.Cu) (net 7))
 (segment (start 97.71 101.25) (end 97.71 99.9543) (width 0.254) (layer F.Cu) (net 7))
 (segment (start 97.2 98.8) (end 97.2 99.6797) (width 0.254) (layer F.Cu) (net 7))
 (segment (start 106.329 94.5) (end 106.329 93.4711) (width 0.1524) (layer F.Cu) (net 22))
 (segment (start 106.7608 93.0393) (end 106.329 93.4711) (width 0.1524) (layer F.Cu) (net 22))
 (segment (start 108.7607 93.0393) (end 106.7608 93.0393) (width 0.1524) (layer F.Cu) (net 22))
 (segment (start 110.6 91.2) (end 108.7607 93.0393) (width 0.1524) (layer F.Cu) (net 22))
 (segment (start 109.0207 93.4711) (end 106.975 93.4711) (width 0.1524) (layer F.Cu) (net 21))
 (segment (start 110.4628 92.029) (end 109.0207 93.4711) (width 0.1524) (layer F.Cu) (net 21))
 (segment (start 111.771 92.029) (end 110.4628 92.029) (width 0.1524) (layer F.Cu) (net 21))
 (segment (start 112.6 91.2) (end 111.771 92.029) (width 0.1524) (layer F.Cu) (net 21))
 (segment (start 106.975 94.5) (end 106.975 93.4711) (width 0.1524) (layer F.Cu) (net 21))
 (via (at 118.1313 92.7946) (size 0.6096) (layers F.Cu B.Cu) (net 20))
 (segment (start 105.9883 95.5289) (end 107.625 95.5289) (width 0.1524) (layer F.Cu) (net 20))
 (segment (start 105.8079 95.3485) (end 105.9883 95.5289) (width 0.1524) (layer F.Cu) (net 20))
 (segment (start 105.8079 93.544) (end 105.8079 95.3485) (width 0.1524) (layer F.Cu) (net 20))
 (segment (start 107.0804 92.2715) (end 105.8079 93.544) (width 0.1524) (layer F.Cu) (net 20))
 (segment (start 108.7136 92.2715) (end 107.0804 92.2715) (width 0.1524) (layer F.Cu) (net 20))
 (segment (start 109.4922 91.4929) (end 108.7136 92.2715) (width 0.1524) (layer F.Cu) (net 20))
 (segment (start 109.4922 91.1097) (end 109.4922 91.4929) (width 0.1524) (layer F.Cu) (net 20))
 (segment (start 110.2309 90.371) (end 109.4922 91.1097) (width 0.1524) (layer F.Cu) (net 20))
 (segment (start 117.1645 90.371) (end 110.2309 90.371) (width 0.1524) (layer F.Cu) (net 20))
 (segment (start 117.65 90.8565) (end 117.1645 90.371) (width 0.1524) (layer F.Cu) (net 20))
 (segment (start 117.65 92.3133) (end 117.65 90.8565) (width 0.1524) (layer F.Cu) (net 20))
 (segment (start 118.1313 92.7946) (end 117.65 92.3133) (width 0.1524) (layer F.Cu) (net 20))
 (segment (start 107.625 94.5) (end 107.625 95.5289) (width 0.1524) (layer F.Cu) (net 20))
 (segment (start 117.35 93.5759) (end 118.1313 92.7946) (width 0.1524) (layer B.Cu) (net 20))
 (segment (start 117.35 96.8354) (end 117.35 93.5759) (width 0.1524) (layer B.Cu) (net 20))
 (segment (start 116.446 97.7394) (end 117.35 96.8354) (width 0.1524) (layer B.Cu) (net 20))
 (segment (start 115.975 97.7394) (end 116.446 97.7394) (width 0.1524) (layer B.Cu) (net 20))
 (segment (start 115.1873 98.5271) (end 115.975 97.7394) (width 0.1524) (layer B.Cu) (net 20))
 (segment (start 115.1873 100.207) (end 115.1873 98.5271) (width 0.1524) (layer B.Cu) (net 20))
 (segment (start 116.23 101.2497) (end 115.1873 100.207) (width 0.1524) (layer B.Cu) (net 20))
 (segment (start 116.23 101.58) (end 116.23 101.2497) (width 0.1524) (layer B.Cu) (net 20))
 (via (at 108.476 96.6526) (size 0.6096) (layers F.Cu B.Cu) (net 19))
 (segment (start 108.476 95.7299) (end 108.476 96.6526) (width 0.1524) (layer F.Cu) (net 19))
 (segment (start 108.275 95.5289) (end 108.476 95.7299) (width 0.1524) (layer F.Cu) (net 19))
 (segment (start 117.7409 102.6091) (end 118.77 101.58) (width 0.1524) (layer B.Cu) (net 19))
 (segment (start 112.8347 102.6091) (end 117.7409 102.6091) (width 0.1524) (layer B.Cu) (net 19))
 (segment (start 111.959 101.7334) (end 112.8347 102.6091) (width 0.1524) (layer B.Cu) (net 19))
 (segment (start 111.959 99.4089) (end 111.959 101.7334) (width 0.1524) (layer B.Cu) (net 19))
 (segment (start 109.6342 97.0841) (end 111.959 99.4089) (width 0.1524) (layer B.Cu) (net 19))
 (segment (start 108.9075 97.0841) (end 109.6342 97.0841) (width 0.1524) (layer B.Cu) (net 19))
 (segment (start 108.476 96.6526) (end 108.9075 97.0841) (width 0.1524) (layer B.Cu) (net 19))
 (segment (start 108.275 94.5) (end 108.275 95.5289) (width 0.1524) (layer F.Cu) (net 19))
 (via (at 114.7398 100.5144) (size 0.6096) (layers F.Cu B.Cu) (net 10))
 (segment (start 114.7398 95.4502) (end 114.7398 100.5144) (width 0.1524) (layer B.Cu) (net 10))
 (segment (start 116.23 93.96) (end 114.7398 95.4502) (width 0.1524) (layer B.Cu) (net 10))
 (segment (start 108.2411 102.145) (end 107.625 101.5289) (width 0.1524) (layer F.Cu) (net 10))
 (segment (start 113.1092 102.145) (end 108.2411 102.145) (width 0.1524) (layer F.Cu) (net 10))
 (segment (start 114.7398 100.5144) (end 113.1092 102.145) (width 0.1524) (layer F.Cu) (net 10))
 (segment (start 107.625 100.5) (end 107.625 101.5289) (width 0.1524) (layer F.Cu) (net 10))
 (segment (start 109.575 100.5) (end 109.575 99.4711) (width 0.1524) (layer F.Cu) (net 11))
 (segment (start 117.6171 95.1129) (end 118.77 93.96) (width 0.1524) (layer F.Cu) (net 11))
 (segment (start 115.3519 95.1129) (end 117.6171 95.1129) (width 0.1524) (layer F.Cu) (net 11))
 (segment (start 110.9937 99.4711) (end 115.3519 95.1129) (width 0.1524) (layer F.Cu) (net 11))
 (segment (start 109.575 99.4711) (end 110.9937 99.4711) (width 0.1524) (layer F.Cu) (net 11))
 (segment (start 113.2589 99.4711) (end 112.175 99.4711) (width 0.1524) (layer F.Cu) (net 15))
 (segment (start 116.23 96.5) (end 113.2589 99.4711) (width 0.1524) (layer F.Cu) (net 15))
 (segment (start 112.175 100.5) (end 112.175 99.4711) (width 0.1524) (layer F.Cu) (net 15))
 (segment (start 115.5516 95.4445) (end 111.525 99.4711) (width 0.1524) (layer F.Cu) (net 14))
 (segment (start 117.7145 95.4445) (end 115.5516 95.4445) (width 0.1524) (layer F.Cu) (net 14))
 (segment (start 118.77 96.5) (end 117.7145 95.4445) (width 0.1524) (layer F.Cu) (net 14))
 (segment (start 111.525 100.5) (end 111.525 99.4711) (width 0.1524) (layer F.Cu) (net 14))
 (segment (start 110.875 100.5) (end 110.875 101.5289) (width 0.1524) (layer F.Cu) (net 13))
 (segment (start 112.539 101.5289) (end 110.875 101.5289) (width 0.1524) (layer F.Cu) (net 13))
 (segment (start 115.0279 99.04) (end 112.539 101.5289) (width 0.1524) (layer F.Cu) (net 13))
 (segment (start 116.23 99.04) (end 115.0279 99.04) (width 0.1524) (layer F.Cu) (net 13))
 (segment (start 110.225 100.5) (end 110.225 101.5289) (width 0.1524) (layer F.Cu) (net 12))
 (segment (start 110.5301 101.834) (end 110.225 101.5289) (width 0.1524) (layer F.Cu) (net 12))
 (segment (start 112.6655 101.834) (end 110.5301 101.834) (width 0.1524) (layer F.Cu) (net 12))
 (segment (start 114.5188 99.9807) (end 112.6655 101.834) (width 0.1524) (layer F.Cu) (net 12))
 (segment (start 114.961 99.9807) (end 114.5188 99.9807) (width 0.1524) (layer F.Cu) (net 12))
 (segment (start 115.089 100.1087) (end 114.961 99.9807) (width 0.1524) (layer F.Cu) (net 12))
 (segment (start 117.7013 100.1087) (end 115.089 100.1087) (width 0.1524) (layer F.Cu) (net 12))
 (segment (start 118.77 99.04) (end 117.7013 100.1087) (width 0.1524) (layer F.Cu) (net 12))
 (via (at 109.4758 97.7652) (size 0.6096) (layers F.Cu B.Cu) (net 8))
 (segment (start 110.225 94.5) (end 110.225 95.5289) (width 0.1524) (layer F.Cu) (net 8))
 (segment (start 98.639 97.266) (end 99.3251 97.266) (width 0.1524) (layer B.Cu) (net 8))
 (segment (start 99.8243 97.7652) (end 109.4758 97.7652) (width 0.1524) (layer B.Cu) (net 8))
 (segment (start 99.3251 97.266) (end 99.8243 97.7652) (width 0.1524) (layer B.Cu) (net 8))
 (segment (start 110.1812 97.0598) (end 109.4758 97.7652) (width 0.1524) (layer F.Cu) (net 8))
 (segment (start 110.1812 96.4927) (end 110.1812 97.0598) (width 0.1524) (layer F.Cu) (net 8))
 (segment (start 110.3621 96.3118) (end 110.1812 96.4927) (width 0.1524) (layer F.Cu) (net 8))
 (segment (start 110.3621 95.666) (end 110.3621 96.3118) (width 0.1524) (layer F.Cu) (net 8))
 (segment (start 110.225 95.5289) (end 110.3621 95.666) (width 0.1524) (layer F.Cu) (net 8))
 (via (at 106.711 99.2282) (size 0.6096) (layers F.Cu B.Cu) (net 9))
 (segment (start 105.6 99.2) (end 105.6 98.5711) (width 0.1524) (layer B.Cu) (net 9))
 (segment (start 111.405 101.5) (end 111.405 100.2711) (width 0.1524) (layer B.Cu) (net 9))
 (segment (start 106.9539 99.4711) (end 106.975 99.4711) (width 0.1524) (layer F.Cu) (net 9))
 (segment (start 106.711 99.2282) (end 106.9539 99.4711) (width 0.1524) (layer F.Cu) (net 9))
 (segment (start 106.975 100.5) (end 106.975 99.4711) (width 0.1524) (layer F.Cu) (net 9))
 (segment (start 105.6 98.5711) (end 106.711 98.5711) (width 0.1524) (layer B.Cu) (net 9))
 (segment (start 106.711 98.5711) (end 106.711 99.2282) (width 0.1524) (layer B.Cu) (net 9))
 (segment (start 111.405 99.2866) (end 111.405 100.2711) (width 0.1524) (layer B.Cu) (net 9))
 (segment (start 110.5122 98.3938) (end 111.405 99.2866) (width 0.1524) (layer B.Cu) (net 9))
 (segment (start 106.8883 98.3938) (end 110.5122 98.3938) (width 0.1524) (layer B.Cu) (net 9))
 (segment (start 106.711 98.5711) (end 106.8883 98.3938) (width 0.1524) (layer B.Cu) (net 9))
 (via (at 111.7286 93.0396) (size 0.6096) (layers F.Cu B.Cu) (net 16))
 (segment (start 111.4971 93.2711) (end 111.7286 93.0396) (width 0.1524) (layer B.Cu) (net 16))
 (segment (start 108.865 93.2711) (end 111.4971 93.2711) (width 0.1524) (layer B.Cu) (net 16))
 (segment (start 112.1601 93.4711) (end 112.175 93.4711) (width 0.1524) (layer F.Cu) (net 16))
 (segment (start 111.7286 93.0396) (end 112.1601 93.4711) (width 0.1524) (layer F.Cu) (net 16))
 (segment (start 112.175 94.5) (end 112.175 93.4711) (width 0.1524) (layer F.Cu) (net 16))
 (segment (start 108.865 94.5) (end 108.865 93.2711) (width 0.1524) (layer B.Cu) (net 16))
 (via (at 110.2839 98.9373) (size 0.6096) (layers F.Cu B.Cu) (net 17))
 (segment (start 110.135 101.5) (end 110.135 100.2711) (width 0.1524) (layer B.Cu) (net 17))
 (segment (start 110.2838 98.9373) (end 110.2839 98.9373) (width 0.1524) (layer B.Cu) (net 17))
 (segment (start 110.2838 100.1223) (end 110.2838 98.9373) (width 0.1524) (layer B.Cu) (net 17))
 (segment (start 110.135 100.2711) (end 110.2838 100.1223) (width 0.1524) (layer B.Cu) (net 17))
 (segment (start 111.525 94.5) (end 111.525 95.5289) (width 0.1524) (layer F.Cu) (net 17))
 (segment (start 111.525 97.6962) (end 111.525 95.5289) (width 0.1524) (layer F.Cu) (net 17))
 (segment (start 110.2839 98.9373) (end 111.525 97.6962) (width 0.1524) (layer F.Cu) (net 17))
 (via (at 110.7149 96.7138) (size 0.6096) (layers F.Cu B.Cu) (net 18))
 (segment (start 109.3888 96.7138) (end 110.7149 96.7138) (width 0.1524) (layer B.Cu) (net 18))
 (segment (start 108.4039 95.7289) (end 109.3888 96.7138) (width 0.1524) (layer B.Cu) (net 18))
 (segment (start 107.595 95.7289) (end 108.4039 95.7289) (width 0.1524) (layer B.Cu) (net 18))
 (segment (start 110.7149 95.689) (end 110.875 95.5289) (width 0.1524) (layer F.Cu) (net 18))
 (segment (start 110.7149 96.7138) (end 110.7149 95.689) (width 0.1524) (layer F.Cu) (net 18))
 (segment (start 110.875 94.5) (end 110.875 95.5289) (width 0.1524) (layer F.Cu) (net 18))
 (segment (start 107.595 94.5) (end 107.595 95.7289) (width 0.1524) (layer B.Cu) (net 18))
 (via (at 107.9141 99.085) (size 0.6096) (layers F.Cu B.Cu) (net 3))
 (segment (start 108.275 99.4459) (end 107.9141 99.085) (width 0.1524) (layer F.Cu) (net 3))
 (segment (start 108.275 100.5) (end 108.275 99.4459) (width 0.1524) (layer F.Cu) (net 3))
 (segment (start 105.878 101.1211) (end 105.5 101.1211) (width 0.1524) (layer B.Cu) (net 3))
 (segment (start 107.9141 99.085) (end 105.878 101.1211) (width 0.1524) (layer B.Cu) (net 3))
 (segment (start 105.5 101.75) (end 105.5 101.1211) (width 0.1524) (layer B.Cu) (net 3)))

